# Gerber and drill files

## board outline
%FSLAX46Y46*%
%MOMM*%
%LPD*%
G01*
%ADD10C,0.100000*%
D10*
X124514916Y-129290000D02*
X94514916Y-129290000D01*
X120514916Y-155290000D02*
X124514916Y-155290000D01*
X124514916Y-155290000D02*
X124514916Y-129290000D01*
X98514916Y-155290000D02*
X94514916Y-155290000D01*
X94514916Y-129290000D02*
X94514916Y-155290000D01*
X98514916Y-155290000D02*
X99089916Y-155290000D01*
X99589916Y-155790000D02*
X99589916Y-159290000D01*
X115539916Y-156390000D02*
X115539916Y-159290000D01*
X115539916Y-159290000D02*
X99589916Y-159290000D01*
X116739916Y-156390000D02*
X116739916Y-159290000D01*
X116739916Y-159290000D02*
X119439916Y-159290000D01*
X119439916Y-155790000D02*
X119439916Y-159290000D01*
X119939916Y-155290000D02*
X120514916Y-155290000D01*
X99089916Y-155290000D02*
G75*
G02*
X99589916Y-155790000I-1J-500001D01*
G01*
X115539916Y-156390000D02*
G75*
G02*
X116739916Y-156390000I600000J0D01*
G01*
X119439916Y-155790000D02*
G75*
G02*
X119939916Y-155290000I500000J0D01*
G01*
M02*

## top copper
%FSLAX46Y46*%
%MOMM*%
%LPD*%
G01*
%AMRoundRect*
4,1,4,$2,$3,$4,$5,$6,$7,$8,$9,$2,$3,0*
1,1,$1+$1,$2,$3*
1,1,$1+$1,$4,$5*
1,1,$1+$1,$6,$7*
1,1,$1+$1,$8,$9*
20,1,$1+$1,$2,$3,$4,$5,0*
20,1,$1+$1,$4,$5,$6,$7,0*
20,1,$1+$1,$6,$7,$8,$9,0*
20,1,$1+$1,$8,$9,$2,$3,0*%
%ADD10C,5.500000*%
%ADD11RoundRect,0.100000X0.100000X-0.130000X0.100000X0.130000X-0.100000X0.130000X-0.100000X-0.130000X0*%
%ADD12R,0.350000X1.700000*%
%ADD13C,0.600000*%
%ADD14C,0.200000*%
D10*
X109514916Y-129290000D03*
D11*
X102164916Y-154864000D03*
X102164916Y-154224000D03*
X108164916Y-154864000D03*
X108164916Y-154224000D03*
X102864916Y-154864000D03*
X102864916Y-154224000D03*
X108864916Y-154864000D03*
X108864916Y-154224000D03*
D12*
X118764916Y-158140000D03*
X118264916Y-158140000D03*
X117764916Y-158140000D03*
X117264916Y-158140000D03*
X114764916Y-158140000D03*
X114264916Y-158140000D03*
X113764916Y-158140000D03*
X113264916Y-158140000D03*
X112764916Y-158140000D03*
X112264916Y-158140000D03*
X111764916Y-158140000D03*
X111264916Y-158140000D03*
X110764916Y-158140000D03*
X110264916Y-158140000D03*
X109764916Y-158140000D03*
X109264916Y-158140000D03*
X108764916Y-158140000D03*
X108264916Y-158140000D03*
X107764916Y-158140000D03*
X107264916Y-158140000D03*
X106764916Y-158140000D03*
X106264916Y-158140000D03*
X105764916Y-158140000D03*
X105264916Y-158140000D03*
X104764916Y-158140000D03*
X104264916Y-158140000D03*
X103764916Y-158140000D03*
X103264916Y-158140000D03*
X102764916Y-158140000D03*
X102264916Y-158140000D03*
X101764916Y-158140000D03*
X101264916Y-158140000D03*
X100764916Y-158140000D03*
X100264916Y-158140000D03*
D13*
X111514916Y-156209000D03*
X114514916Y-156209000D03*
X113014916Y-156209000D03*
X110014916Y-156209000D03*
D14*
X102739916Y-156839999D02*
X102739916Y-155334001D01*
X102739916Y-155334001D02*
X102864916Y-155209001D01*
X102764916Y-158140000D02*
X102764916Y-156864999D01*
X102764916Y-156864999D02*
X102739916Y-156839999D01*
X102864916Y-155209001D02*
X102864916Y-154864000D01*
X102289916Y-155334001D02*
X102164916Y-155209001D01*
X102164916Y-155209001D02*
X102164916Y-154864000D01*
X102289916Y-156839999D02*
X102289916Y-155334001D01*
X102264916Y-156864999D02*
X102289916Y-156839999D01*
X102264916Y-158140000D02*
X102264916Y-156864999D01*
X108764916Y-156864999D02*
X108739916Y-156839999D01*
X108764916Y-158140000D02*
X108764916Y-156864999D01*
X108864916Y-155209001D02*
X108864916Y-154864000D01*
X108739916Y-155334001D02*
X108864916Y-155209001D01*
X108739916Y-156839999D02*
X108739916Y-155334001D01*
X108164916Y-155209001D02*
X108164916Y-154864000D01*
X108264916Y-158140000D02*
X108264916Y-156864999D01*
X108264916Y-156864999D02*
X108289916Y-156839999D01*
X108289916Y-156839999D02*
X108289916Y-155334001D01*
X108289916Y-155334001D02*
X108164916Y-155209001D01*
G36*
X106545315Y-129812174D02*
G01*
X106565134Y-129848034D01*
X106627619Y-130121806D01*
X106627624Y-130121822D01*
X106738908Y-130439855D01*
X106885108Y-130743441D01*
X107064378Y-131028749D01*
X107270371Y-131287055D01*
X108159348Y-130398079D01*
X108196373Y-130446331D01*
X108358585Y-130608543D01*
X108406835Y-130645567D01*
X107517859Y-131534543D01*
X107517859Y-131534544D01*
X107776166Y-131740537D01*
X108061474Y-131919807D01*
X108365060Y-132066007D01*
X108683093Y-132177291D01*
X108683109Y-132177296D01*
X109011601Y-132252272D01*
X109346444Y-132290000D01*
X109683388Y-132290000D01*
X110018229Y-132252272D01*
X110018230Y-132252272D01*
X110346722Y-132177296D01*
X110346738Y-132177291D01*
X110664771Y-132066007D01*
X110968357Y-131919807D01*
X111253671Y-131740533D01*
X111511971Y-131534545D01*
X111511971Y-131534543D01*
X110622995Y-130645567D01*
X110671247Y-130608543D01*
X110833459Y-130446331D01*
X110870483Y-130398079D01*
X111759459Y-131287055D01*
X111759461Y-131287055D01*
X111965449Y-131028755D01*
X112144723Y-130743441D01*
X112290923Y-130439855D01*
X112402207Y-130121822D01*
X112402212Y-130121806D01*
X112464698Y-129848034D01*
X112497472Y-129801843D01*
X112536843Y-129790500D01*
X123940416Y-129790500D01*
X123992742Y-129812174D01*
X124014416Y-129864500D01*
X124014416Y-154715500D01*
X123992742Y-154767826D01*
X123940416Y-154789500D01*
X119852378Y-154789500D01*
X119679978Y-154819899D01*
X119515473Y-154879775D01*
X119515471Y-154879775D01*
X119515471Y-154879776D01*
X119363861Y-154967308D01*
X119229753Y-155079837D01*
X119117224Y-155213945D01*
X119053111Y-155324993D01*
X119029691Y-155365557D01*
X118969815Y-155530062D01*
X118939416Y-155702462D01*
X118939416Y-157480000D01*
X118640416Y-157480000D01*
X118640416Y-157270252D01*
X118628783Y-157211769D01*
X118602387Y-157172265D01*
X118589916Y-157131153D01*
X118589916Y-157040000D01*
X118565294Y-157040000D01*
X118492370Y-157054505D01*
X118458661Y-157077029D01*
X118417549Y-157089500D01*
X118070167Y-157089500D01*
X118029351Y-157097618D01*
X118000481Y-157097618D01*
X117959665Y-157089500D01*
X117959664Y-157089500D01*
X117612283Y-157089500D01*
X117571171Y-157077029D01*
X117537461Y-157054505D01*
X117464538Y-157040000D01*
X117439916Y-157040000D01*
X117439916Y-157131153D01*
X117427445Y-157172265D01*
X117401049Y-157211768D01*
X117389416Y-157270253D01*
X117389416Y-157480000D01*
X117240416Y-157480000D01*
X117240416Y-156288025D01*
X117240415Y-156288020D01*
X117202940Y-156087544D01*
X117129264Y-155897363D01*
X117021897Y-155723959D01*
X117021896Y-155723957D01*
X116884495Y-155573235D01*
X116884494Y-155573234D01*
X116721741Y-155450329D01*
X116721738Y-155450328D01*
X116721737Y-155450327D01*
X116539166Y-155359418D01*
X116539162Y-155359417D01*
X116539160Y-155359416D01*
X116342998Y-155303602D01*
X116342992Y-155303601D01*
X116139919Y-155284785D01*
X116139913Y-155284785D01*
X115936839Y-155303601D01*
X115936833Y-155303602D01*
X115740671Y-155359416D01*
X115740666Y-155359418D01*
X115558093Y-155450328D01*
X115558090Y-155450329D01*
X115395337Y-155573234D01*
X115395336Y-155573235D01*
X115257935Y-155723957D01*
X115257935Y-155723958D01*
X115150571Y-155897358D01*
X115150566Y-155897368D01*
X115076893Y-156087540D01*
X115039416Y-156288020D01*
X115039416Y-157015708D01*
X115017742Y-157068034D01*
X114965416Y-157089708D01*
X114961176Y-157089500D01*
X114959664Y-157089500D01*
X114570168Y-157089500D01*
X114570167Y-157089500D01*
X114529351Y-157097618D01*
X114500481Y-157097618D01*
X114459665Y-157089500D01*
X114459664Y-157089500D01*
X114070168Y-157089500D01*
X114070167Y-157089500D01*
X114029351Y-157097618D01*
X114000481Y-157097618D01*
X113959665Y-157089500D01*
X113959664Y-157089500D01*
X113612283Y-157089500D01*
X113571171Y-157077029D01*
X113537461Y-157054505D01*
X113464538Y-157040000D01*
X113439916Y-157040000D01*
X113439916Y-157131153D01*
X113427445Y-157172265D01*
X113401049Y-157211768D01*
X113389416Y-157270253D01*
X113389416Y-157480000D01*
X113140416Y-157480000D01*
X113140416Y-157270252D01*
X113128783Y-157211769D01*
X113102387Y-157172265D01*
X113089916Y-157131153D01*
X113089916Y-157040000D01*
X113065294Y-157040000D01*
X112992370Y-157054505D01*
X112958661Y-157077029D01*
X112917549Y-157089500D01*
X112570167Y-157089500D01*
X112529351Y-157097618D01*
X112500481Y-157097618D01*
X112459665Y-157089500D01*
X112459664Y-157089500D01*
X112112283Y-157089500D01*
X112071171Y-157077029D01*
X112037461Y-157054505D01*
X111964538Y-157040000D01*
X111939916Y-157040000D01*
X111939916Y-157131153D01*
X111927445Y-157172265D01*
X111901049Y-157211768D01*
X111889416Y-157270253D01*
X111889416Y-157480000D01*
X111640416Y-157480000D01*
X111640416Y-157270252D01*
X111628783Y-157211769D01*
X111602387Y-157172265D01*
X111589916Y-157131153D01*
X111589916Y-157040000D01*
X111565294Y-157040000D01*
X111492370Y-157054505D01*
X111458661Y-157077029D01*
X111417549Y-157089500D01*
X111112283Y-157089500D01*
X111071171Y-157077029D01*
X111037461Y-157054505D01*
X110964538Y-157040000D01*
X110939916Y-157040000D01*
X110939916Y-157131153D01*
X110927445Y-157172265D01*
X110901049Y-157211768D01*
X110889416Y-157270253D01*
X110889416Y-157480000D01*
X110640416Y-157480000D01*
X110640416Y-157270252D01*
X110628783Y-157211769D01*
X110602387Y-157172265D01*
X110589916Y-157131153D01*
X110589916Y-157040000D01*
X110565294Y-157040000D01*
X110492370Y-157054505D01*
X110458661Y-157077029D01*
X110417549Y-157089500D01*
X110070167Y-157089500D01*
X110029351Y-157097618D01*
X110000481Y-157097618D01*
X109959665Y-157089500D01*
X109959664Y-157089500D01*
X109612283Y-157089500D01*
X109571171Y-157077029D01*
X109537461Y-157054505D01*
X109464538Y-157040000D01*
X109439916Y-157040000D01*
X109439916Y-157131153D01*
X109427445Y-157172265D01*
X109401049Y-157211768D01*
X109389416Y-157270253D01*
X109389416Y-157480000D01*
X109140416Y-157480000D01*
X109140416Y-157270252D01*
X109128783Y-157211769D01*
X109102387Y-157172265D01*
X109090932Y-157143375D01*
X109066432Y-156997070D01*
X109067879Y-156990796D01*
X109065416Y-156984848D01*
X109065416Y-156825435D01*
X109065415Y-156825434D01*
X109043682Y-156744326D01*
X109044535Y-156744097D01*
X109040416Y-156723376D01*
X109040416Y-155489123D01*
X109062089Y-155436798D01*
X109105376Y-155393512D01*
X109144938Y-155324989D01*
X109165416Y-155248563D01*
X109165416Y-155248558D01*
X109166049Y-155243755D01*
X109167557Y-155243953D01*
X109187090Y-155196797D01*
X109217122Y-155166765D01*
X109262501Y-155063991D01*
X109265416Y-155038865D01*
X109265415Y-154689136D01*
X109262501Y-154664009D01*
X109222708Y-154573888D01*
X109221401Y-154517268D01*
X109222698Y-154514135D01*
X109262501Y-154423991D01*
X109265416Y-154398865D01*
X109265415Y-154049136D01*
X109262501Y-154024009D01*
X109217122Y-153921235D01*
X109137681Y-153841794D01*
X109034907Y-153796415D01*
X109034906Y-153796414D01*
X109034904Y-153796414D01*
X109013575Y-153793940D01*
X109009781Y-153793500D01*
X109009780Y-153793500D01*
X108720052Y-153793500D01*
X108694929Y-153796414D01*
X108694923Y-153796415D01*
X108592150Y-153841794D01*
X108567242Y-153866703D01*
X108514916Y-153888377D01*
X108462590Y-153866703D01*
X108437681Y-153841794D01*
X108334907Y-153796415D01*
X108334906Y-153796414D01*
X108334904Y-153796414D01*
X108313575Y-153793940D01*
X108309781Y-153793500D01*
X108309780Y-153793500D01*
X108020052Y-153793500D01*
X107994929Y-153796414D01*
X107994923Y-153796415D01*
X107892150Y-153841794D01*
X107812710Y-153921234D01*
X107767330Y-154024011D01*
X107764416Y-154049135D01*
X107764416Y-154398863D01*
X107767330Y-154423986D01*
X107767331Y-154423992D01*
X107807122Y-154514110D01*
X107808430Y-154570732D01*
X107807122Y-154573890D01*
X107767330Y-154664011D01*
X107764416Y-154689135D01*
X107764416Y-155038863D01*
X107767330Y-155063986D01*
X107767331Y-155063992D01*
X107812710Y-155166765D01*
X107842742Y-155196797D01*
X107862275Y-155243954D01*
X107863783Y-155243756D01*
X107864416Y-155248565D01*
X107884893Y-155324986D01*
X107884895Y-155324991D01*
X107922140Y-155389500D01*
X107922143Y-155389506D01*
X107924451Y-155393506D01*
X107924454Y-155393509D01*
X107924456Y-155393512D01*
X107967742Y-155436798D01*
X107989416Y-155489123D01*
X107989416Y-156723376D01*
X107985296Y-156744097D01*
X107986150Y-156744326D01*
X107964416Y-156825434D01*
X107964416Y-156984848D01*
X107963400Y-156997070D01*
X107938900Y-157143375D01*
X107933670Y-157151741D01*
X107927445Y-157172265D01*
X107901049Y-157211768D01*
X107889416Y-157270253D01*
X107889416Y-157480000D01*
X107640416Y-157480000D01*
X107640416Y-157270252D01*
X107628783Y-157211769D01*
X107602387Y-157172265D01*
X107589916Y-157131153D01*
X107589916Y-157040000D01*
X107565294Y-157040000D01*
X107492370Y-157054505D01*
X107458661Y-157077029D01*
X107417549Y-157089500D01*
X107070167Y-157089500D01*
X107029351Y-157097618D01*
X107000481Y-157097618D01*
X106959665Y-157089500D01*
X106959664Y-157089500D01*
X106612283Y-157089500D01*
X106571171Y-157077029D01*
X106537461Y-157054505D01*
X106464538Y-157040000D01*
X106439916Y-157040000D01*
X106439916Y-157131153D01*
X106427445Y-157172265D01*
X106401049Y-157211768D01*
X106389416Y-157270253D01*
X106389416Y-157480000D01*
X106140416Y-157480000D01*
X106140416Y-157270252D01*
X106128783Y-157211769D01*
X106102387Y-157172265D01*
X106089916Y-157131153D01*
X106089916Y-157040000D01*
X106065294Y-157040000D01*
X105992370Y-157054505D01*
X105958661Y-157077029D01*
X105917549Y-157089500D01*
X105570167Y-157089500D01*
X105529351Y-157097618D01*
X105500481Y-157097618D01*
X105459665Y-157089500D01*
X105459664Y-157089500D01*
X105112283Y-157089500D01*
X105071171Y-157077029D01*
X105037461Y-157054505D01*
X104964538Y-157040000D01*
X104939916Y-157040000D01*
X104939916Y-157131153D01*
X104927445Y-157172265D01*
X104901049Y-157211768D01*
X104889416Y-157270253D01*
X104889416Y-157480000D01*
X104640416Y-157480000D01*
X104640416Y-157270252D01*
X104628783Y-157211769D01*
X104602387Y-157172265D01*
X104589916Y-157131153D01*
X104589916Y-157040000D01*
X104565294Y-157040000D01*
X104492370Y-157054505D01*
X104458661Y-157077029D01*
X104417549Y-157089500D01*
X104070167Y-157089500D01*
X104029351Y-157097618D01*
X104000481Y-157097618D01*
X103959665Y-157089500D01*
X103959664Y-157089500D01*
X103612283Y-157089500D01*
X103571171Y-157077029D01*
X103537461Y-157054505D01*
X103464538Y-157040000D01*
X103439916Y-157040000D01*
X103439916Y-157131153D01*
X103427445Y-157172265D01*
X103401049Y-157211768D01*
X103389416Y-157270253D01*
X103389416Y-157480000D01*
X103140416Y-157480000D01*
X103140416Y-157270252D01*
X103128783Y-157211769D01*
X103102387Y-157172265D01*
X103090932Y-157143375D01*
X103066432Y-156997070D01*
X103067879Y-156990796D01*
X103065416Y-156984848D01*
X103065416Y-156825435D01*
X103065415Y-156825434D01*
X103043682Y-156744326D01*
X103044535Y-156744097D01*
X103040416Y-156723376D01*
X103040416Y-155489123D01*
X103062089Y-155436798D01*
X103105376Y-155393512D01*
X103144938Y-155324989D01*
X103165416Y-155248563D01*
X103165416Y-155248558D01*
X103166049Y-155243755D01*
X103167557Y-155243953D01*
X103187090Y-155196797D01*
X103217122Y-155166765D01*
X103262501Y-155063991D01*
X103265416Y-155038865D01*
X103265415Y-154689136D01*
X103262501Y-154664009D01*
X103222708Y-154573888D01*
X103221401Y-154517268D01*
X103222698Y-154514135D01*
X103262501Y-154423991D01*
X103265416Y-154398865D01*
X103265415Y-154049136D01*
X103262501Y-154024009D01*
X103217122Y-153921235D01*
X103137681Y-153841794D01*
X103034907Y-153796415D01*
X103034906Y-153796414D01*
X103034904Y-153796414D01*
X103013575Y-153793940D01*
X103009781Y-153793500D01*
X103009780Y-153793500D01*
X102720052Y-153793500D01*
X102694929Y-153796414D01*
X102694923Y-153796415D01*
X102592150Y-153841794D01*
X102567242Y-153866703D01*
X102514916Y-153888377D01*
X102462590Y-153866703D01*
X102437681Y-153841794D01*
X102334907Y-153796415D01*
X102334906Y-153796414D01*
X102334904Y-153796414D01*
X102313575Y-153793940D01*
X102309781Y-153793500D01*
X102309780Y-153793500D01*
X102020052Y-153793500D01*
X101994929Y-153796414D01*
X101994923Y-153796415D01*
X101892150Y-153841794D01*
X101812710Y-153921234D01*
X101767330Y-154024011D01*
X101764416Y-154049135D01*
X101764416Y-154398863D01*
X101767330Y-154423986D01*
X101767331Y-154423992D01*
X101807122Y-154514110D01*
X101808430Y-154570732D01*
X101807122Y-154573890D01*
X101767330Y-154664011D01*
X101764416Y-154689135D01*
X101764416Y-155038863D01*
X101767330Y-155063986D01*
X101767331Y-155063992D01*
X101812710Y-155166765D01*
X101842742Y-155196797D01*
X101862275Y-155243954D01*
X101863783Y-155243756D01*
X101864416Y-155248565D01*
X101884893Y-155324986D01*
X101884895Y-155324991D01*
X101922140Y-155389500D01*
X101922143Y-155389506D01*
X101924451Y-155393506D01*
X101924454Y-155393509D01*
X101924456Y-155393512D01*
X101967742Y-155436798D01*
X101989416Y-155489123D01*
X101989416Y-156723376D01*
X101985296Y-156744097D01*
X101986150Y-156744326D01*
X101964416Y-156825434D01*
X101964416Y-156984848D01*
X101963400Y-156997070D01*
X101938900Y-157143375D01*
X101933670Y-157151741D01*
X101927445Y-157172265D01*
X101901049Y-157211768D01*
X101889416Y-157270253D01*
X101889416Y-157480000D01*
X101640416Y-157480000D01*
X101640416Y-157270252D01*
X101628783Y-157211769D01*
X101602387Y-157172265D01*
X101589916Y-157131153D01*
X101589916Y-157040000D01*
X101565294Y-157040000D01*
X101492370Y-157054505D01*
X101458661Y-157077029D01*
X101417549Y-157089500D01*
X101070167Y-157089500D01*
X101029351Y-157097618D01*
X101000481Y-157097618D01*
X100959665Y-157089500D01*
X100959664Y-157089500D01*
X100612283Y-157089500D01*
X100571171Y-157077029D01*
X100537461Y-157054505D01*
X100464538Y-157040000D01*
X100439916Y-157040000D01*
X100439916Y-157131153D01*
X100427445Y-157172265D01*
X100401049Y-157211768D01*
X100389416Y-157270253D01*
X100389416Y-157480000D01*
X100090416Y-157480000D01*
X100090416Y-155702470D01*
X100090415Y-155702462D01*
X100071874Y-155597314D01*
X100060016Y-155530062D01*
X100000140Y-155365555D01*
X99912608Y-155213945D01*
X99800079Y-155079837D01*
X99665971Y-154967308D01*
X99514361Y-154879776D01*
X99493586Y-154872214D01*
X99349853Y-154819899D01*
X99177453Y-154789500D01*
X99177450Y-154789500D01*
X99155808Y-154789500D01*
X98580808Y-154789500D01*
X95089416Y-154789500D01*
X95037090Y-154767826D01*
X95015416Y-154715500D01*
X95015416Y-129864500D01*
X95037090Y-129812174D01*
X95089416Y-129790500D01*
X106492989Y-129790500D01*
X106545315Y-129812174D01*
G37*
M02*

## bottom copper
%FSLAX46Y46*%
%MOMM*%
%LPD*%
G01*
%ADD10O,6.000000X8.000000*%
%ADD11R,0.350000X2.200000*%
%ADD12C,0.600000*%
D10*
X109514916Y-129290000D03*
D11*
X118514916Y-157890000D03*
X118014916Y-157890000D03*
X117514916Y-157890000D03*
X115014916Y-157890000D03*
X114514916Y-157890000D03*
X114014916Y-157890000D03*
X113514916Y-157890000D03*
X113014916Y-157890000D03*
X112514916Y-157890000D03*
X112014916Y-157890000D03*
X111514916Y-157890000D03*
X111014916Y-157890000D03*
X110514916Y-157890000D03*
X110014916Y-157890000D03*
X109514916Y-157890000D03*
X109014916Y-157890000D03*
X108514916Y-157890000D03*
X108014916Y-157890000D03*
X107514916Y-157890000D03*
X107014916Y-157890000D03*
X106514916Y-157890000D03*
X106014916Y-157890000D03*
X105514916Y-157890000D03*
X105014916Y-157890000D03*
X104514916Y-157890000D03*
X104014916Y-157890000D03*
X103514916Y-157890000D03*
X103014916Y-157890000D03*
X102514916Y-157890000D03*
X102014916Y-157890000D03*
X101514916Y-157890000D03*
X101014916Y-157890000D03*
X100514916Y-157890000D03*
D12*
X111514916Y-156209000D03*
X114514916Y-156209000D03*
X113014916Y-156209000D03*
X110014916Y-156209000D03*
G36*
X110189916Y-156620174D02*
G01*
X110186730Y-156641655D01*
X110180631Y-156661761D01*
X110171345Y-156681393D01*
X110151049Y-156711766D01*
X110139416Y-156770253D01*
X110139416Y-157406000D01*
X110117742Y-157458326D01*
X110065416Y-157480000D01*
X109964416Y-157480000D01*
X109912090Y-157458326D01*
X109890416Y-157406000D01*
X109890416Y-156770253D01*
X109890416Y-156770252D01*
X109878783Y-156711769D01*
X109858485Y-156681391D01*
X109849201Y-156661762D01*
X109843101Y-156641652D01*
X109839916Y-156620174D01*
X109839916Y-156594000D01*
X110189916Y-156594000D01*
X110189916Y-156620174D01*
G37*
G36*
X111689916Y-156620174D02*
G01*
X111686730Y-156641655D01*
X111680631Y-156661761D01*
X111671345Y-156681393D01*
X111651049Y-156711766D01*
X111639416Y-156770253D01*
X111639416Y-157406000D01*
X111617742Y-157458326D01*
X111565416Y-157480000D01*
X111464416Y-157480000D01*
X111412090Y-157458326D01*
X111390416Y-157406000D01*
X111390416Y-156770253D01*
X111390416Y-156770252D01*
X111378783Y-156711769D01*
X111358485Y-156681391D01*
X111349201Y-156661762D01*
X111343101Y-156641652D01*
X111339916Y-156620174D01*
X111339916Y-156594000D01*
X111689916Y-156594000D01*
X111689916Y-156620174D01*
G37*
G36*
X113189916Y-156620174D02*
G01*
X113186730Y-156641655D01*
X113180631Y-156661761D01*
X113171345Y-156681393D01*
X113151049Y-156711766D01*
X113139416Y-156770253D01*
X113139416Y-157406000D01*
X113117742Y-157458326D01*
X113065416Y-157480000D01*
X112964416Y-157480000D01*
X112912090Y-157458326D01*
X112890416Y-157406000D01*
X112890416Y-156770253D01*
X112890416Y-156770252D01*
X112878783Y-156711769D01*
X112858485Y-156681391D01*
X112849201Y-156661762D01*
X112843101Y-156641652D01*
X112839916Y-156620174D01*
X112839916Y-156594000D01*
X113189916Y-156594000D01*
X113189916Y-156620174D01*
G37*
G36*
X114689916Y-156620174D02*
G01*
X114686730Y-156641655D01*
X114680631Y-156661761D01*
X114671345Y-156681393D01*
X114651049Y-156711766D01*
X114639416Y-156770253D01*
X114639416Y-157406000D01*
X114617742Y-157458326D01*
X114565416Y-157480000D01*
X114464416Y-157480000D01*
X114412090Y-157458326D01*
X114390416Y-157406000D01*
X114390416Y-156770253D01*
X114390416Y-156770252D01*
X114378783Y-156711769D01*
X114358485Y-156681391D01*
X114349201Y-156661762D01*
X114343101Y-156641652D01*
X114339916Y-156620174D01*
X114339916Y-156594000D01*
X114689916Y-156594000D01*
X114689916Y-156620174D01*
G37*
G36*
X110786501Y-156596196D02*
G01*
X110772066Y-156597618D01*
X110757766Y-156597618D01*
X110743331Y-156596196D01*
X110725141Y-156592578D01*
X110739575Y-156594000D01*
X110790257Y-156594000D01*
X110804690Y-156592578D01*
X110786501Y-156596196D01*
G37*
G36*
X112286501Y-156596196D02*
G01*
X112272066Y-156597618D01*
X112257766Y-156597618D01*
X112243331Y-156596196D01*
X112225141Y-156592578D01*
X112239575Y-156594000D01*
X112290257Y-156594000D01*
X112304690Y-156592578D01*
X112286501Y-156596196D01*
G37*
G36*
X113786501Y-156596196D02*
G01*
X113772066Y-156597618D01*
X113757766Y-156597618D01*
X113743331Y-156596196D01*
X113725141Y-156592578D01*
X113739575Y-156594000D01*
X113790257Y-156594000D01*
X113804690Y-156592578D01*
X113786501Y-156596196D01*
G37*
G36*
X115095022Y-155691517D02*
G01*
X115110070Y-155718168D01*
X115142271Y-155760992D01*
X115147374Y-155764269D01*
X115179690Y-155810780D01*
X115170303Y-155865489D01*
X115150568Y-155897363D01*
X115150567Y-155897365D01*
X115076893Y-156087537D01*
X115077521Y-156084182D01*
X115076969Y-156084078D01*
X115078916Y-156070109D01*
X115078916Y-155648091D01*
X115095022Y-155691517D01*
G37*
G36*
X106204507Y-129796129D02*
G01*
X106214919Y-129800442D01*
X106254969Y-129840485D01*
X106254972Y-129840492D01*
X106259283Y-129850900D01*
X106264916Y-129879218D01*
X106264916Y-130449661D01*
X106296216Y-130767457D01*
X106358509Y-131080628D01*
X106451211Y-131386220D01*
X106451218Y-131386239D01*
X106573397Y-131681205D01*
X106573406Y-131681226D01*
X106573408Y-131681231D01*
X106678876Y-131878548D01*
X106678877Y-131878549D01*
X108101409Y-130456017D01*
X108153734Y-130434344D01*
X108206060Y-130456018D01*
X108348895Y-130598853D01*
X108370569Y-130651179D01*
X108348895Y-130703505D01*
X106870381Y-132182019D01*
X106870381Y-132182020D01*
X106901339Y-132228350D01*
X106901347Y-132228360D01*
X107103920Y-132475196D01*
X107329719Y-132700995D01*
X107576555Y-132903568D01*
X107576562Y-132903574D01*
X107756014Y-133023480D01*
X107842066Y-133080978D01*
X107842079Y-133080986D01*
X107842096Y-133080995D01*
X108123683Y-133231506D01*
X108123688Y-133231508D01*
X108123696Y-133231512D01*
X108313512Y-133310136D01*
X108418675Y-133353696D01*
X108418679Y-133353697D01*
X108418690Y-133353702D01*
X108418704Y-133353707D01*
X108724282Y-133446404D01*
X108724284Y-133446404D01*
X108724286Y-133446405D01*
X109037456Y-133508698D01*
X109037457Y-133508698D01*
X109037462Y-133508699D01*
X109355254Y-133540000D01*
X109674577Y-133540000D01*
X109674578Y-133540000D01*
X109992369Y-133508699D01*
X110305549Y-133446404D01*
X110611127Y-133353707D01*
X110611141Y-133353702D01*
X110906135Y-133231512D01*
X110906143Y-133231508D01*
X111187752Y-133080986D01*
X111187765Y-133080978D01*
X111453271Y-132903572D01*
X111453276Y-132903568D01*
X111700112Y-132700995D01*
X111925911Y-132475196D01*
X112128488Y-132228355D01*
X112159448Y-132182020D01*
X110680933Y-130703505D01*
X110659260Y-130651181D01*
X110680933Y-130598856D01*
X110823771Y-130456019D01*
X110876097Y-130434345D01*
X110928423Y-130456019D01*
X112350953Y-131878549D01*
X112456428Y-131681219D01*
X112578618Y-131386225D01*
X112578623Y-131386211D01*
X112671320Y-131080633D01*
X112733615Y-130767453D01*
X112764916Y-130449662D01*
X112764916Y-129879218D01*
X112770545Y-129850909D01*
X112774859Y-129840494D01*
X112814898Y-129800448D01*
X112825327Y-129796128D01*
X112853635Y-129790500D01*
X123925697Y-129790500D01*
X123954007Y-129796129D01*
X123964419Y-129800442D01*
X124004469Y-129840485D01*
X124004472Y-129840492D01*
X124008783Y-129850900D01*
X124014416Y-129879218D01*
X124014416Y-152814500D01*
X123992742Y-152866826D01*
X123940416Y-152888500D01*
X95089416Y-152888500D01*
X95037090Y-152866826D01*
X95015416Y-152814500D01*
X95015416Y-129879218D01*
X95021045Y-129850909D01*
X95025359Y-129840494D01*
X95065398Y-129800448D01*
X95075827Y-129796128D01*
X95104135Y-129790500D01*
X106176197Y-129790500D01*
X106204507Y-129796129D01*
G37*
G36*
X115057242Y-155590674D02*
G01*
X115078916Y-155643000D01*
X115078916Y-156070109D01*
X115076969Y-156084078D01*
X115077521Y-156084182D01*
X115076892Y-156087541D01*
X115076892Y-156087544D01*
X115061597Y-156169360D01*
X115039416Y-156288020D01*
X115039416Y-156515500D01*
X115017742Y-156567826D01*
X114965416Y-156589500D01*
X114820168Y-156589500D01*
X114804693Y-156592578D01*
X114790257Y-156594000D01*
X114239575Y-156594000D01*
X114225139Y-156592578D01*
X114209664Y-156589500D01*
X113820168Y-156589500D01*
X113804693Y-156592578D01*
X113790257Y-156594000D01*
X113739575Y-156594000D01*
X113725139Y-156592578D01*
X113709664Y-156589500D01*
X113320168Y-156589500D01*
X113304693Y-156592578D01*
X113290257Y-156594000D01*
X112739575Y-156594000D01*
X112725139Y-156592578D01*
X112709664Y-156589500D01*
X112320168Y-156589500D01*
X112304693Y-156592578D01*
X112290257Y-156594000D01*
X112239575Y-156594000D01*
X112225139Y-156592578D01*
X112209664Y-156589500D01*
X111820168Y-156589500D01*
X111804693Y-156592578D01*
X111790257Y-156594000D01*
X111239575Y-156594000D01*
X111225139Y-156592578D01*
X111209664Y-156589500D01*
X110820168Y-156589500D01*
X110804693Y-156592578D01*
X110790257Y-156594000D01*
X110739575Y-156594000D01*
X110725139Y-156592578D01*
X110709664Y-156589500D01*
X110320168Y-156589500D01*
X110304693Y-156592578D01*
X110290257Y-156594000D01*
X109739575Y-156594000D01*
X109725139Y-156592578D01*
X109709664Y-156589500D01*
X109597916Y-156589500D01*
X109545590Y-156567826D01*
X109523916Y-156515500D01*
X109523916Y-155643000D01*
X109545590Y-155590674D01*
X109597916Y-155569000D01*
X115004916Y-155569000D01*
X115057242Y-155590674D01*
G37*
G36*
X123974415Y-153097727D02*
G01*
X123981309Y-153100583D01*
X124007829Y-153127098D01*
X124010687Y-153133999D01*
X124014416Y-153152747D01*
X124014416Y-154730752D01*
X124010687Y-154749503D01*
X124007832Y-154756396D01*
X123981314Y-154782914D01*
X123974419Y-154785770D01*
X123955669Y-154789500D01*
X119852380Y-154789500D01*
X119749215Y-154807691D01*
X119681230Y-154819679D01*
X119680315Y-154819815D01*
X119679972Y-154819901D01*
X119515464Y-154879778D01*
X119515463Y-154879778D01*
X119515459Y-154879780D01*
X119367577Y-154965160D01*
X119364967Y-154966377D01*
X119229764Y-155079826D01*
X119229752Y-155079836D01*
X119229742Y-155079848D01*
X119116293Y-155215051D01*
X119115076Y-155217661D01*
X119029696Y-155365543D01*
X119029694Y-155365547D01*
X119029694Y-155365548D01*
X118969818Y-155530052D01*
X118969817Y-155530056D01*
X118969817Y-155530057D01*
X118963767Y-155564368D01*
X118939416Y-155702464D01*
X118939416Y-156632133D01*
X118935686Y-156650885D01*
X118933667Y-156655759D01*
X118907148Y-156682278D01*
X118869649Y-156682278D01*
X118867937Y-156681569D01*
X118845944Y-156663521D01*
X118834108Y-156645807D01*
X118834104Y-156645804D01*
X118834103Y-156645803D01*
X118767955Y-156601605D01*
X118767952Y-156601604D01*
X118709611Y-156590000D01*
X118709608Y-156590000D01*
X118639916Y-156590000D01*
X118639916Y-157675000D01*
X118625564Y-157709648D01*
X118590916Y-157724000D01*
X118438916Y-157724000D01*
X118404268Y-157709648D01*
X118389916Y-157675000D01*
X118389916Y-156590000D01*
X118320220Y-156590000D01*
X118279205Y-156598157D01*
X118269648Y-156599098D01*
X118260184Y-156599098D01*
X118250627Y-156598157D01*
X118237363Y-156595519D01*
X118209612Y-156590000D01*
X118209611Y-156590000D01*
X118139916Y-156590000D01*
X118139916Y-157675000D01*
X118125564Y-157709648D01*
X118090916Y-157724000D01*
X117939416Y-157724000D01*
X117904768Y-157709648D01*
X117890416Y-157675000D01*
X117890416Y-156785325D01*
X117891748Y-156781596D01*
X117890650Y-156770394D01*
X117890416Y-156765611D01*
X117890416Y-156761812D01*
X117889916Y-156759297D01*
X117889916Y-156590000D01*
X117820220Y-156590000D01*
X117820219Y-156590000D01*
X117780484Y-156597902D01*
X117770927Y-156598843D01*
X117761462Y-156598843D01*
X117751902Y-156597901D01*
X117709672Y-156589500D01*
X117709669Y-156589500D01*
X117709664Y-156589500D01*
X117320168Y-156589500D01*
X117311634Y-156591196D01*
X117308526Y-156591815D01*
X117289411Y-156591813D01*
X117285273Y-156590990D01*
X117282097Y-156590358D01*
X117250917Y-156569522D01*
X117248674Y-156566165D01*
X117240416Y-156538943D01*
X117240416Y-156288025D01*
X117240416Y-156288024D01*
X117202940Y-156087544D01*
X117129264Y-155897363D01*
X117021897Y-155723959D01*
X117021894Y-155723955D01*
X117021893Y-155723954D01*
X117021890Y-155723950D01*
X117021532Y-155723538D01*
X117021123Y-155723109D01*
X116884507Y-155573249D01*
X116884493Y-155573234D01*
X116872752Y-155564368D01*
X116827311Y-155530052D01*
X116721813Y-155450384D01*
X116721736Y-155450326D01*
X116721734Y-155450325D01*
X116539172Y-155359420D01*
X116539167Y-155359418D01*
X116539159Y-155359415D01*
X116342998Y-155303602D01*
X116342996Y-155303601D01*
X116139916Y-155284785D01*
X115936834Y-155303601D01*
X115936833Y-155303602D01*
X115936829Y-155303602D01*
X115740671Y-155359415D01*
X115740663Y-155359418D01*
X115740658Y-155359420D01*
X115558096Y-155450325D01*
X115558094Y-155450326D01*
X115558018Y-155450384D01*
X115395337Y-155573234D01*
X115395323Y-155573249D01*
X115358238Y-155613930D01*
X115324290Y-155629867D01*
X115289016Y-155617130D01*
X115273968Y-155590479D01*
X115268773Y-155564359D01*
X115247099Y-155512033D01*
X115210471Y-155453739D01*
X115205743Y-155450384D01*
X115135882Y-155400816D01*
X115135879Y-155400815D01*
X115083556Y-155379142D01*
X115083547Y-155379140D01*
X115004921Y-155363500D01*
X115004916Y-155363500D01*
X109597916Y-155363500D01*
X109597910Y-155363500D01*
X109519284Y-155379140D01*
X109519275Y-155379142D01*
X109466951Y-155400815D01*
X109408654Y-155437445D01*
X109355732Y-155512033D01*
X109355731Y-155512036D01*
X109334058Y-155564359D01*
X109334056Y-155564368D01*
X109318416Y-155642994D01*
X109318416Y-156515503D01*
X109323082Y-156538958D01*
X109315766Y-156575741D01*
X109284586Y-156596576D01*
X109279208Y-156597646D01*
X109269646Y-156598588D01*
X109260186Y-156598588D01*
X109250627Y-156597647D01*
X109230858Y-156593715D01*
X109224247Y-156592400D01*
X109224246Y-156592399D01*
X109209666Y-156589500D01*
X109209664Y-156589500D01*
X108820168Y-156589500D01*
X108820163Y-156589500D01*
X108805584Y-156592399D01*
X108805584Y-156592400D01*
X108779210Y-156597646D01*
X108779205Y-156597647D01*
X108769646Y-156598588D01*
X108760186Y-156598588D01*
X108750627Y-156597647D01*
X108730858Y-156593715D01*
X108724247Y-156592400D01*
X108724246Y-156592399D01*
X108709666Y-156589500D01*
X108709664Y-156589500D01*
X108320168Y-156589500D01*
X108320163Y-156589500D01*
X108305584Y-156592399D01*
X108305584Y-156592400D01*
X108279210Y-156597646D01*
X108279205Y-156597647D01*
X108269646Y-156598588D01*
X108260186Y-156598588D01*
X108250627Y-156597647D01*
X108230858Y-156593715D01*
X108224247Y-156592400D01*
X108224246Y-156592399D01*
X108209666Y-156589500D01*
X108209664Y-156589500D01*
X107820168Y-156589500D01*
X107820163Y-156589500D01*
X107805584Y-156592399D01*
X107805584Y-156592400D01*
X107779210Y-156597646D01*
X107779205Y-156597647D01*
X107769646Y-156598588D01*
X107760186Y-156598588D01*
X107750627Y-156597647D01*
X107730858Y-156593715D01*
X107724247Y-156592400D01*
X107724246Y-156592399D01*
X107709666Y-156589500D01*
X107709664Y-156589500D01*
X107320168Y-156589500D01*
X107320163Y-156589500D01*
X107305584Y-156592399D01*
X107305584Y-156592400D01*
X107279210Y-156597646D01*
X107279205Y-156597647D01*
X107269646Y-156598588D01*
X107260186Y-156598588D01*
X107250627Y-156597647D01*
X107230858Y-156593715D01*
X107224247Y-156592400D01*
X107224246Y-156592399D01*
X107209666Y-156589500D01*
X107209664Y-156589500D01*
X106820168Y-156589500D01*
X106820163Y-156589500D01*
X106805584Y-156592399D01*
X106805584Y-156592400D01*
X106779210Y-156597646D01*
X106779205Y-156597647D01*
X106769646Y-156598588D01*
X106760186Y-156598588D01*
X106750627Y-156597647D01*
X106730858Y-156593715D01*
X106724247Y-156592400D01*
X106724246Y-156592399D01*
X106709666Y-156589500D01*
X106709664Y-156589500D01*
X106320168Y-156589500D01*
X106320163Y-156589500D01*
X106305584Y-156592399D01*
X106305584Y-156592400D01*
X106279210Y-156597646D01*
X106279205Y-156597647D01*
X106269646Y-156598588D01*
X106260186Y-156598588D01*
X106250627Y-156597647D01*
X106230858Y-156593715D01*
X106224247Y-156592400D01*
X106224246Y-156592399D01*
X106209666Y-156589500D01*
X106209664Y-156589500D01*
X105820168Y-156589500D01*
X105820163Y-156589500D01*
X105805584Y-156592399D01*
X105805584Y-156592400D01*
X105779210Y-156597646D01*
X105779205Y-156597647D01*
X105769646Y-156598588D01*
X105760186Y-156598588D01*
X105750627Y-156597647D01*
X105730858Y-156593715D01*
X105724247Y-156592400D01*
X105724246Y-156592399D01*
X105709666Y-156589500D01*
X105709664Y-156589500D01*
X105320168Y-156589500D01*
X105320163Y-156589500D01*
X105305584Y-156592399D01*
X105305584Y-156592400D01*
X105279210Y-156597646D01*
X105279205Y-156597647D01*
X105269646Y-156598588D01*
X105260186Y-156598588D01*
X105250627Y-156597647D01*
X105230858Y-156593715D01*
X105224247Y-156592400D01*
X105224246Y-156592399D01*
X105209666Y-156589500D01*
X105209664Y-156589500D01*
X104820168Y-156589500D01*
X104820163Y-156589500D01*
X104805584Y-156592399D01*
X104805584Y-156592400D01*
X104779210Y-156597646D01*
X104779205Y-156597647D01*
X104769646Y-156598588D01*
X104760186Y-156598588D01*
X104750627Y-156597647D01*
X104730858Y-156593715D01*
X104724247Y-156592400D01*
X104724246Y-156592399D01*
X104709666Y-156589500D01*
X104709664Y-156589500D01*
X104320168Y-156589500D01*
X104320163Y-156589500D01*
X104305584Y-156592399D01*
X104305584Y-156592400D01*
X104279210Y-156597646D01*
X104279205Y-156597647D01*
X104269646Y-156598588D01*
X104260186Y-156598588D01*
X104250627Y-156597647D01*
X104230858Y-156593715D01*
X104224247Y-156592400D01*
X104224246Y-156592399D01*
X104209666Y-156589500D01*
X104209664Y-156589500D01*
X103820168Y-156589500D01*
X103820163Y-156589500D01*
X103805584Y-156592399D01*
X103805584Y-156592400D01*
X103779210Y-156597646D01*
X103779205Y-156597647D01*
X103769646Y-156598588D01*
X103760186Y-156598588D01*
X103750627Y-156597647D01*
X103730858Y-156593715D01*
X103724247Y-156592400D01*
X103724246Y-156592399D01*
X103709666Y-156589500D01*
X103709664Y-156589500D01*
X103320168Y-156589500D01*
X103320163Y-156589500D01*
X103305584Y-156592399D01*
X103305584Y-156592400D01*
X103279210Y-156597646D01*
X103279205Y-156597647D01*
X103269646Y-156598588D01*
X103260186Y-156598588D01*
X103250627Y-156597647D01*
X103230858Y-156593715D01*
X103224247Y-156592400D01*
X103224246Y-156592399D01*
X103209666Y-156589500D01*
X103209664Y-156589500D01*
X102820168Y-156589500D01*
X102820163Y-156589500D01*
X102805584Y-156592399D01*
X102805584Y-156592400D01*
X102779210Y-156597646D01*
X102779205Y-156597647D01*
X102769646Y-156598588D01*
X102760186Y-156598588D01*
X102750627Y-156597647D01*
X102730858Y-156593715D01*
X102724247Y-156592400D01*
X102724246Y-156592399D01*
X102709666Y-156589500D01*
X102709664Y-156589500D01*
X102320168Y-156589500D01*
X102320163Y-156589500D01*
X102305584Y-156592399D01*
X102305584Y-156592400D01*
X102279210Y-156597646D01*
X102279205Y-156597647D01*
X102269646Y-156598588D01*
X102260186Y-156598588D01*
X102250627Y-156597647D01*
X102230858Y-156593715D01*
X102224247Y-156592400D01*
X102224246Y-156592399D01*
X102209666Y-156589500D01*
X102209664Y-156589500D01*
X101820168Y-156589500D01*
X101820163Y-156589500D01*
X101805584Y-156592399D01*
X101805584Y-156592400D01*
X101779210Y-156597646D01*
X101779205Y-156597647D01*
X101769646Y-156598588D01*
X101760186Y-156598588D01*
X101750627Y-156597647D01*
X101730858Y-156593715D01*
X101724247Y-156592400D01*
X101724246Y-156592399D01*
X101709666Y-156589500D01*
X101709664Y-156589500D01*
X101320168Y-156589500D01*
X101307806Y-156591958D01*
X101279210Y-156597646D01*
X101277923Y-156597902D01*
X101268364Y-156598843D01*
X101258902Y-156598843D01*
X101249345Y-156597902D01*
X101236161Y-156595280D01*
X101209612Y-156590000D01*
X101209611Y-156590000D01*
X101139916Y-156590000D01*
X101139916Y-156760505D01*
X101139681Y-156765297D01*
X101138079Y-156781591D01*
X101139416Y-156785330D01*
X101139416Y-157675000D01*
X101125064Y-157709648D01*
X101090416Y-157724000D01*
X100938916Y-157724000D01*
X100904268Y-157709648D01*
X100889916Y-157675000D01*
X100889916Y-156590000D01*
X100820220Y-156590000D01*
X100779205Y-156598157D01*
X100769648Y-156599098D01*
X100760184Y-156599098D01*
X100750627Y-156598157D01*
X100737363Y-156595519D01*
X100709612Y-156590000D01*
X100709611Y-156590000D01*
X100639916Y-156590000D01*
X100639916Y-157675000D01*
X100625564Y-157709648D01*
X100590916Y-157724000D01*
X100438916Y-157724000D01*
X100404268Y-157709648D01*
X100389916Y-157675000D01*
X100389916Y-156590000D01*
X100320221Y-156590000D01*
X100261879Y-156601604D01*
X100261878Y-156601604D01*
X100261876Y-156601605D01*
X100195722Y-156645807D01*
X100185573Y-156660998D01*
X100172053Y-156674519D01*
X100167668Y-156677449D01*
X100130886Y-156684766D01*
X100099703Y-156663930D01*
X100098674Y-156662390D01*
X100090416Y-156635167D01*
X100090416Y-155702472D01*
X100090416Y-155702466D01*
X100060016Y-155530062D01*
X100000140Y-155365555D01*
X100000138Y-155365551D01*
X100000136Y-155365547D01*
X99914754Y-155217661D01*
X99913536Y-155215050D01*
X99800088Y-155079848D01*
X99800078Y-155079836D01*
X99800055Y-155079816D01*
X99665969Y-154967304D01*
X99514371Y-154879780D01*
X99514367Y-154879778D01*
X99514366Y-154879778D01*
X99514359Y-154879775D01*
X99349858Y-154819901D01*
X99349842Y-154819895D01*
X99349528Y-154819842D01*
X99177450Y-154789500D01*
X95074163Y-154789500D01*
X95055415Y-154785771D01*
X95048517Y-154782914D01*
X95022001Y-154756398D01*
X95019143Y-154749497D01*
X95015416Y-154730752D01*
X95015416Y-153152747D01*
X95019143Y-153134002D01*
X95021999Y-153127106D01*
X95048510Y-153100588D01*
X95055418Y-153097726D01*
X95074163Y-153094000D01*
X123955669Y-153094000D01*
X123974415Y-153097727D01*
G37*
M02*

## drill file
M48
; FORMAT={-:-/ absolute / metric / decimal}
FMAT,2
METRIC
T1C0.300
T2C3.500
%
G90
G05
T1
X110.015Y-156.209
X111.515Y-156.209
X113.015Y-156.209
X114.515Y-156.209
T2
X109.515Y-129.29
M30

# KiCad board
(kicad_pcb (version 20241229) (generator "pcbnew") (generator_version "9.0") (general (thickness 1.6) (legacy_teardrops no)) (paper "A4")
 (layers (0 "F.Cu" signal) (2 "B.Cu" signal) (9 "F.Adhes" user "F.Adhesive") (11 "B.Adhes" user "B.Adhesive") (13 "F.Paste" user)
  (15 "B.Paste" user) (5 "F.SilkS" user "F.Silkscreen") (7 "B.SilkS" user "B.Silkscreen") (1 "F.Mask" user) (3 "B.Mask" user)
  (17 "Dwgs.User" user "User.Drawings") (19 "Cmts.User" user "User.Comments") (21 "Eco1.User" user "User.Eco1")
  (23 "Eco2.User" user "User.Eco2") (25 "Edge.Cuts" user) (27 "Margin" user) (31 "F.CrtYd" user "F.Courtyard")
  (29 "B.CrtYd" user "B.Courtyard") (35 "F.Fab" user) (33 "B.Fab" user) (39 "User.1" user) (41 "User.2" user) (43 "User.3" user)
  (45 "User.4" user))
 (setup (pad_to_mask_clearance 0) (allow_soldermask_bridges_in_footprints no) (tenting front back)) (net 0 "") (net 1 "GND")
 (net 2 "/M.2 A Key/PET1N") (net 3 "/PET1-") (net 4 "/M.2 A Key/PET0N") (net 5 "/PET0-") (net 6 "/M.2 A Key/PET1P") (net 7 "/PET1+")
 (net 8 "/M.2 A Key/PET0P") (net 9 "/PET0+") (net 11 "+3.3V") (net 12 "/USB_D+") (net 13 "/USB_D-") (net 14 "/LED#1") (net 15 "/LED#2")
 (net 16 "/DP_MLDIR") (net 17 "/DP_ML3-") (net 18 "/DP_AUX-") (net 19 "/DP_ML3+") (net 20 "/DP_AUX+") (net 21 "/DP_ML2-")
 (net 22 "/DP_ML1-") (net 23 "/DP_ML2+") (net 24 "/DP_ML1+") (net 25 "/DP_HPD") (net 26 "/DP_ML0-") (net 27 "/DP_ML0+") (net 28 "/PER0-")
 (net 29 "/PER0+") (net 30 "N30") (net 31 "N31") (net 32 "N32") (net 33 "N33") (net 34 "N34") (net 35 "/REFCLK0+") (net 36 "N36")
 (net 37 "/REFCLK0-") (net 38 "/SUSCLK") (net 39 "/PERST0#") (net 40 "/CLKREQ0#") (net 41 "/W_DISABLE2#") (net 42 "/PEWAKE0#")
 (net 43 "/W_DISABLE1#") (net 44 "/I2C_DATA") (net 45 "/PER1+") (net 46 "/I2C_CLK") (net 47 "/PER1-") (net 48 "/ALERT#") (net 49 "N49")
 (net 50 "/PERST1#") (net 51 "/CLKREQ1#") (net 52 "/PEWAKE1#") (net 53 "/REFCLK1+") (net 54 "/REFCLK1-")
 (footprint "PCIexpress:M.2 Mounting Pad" (layer "F.Cu") (at 109.514916 129.29)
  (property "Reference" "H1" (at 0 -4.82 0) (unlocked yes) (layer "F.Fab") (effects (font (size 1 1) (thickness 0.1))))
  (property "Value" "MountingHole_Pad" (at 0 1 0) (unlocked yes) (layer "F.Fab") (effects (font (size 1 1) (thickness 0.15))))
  (pad "1" thru_hole circle (at 0 0) (size 5.5 5.5) (drill 3.5) (layers "*.Cu" "*.Mask") (remove_unused_layers no) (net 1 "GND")
   (padstack (mode front_inner_back)
    (layer "Inner" (shape circle) (size 5.5 5.5) (zone_connect -1))
    (layer "B.Cu" (shape oval) (size 6 8) (thermal_bridge_angle 45) (zone_connect -1)))))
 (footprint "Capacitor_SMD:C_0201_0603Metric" (layer "F.Cu") (at 102.164916 154.544 90)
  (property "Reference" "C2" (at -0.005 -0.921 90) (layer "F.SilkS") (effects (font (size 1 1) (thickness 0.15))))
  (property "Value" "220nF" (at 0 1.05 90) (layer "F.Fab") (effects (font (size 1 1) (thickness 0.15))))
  (pad "" smd roundrect (at -0.345 0 90) (size 0.318 0.36) (layers "F.Paste") (roundrect_rratio 0.25))
  (pad "" smd roundrect (at 0.345 0 90) (size 0.318 0.36) (layers "F.Paste") (roundrect_rratio 0.25))
  (pad "1" smd roundrect (at -0.32 0 90) (size 0.46 0.4) (layers "F.Cu" "F.Mask") (roundrect_rratio 0.25) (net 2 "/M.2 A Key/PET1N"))
  (pad "2" smd roundrect (at 0.32 0 90) (size 0.46 0.4) (layers "F.Cu" "F.Mask") (roundrect_rratio 0.25) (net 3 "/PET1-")))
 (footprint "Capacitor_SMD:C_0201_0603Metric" (layer "F.Cu") (at 108.164916 154.544 90)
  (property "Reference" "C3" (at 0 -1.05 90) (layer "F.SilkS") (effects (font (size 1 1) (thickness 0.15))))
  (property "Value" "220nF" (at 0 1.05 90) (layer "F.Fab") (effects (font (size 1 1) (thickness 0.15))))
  (pad "" smd roundrect (at -0.345 0 90) (size 0.318 0.36) (layers "F.Paste") (roundrect_rratio 0.25))
  (pad "" smd roundrect (at 0.345 0 90) (size 0.318 0.36) (layers "F.Paste") (roundrect_rratio 0.25))
  (pad "1" smd roundrect (at -0.32 0 90) (size 0.46 0.4) (layers "F.Cu" "F.Mask") (roundrect_rratio 0.25) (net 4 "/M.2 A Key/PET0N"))
  (pad "2" smd roundrect (at 0.32 0 90) (size 0.46 0.4) (layers "F.Cu" "F.Mask") (roundrect_rratio 0.25) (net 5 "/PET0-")))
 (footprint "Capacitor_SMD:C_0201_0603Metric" (layer "F.Cu") (at 102.864916 154.544 90)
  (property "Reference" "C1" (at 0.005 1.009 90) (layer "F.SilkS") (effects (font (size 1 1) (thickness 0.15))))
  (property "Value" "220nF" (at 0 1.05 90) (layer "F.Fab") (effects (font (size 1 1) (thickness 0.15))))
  (pad "" smd roundrect (at -0.345 0 90) (size 0.318 0.36) (layers "F.Paste") (roundrect_rratio 0.25))
  (pad "" smd roundrect (at 0.345 0 90) (size 0.318 0.36) (layers "F.Paste") (roundrect_rratio 0.25))
  (pad "1" smd roundrect (at -0.32 0 90) (size 0.46 0.4) (layers "F.Cu" "F.Mask") (roundrect_rratio 0.25) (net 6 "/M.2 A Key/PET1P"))
  (pad "2" smd roundrect (at 0.32 0 90) (size 0.46 0.4) (layers "F.Cu" "F.Mask") (roundrect_rratio 0.25) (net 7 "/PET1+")))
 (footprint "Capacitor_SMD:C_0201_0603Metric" (layer "F.Cu") (at 108.864916 154.544 90)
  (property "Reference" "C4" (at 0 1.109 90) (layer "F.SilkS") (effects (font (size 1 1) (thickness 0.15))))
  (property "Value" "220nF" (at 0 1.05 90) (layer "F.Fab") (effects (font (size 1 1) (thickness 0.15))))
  (pad "" smd roundrect (at -0.345 0 90) (size 0.318 0.36) (layers "F.Paste") (roundrect_rratio 0.25))
  (pad "" smd roundrect (at 0.345 0 90) (size 0.318 0.36) (layers "F.Paste") (roundrect_rratio 0.25))
  (pad "1" smd roundrect (at -0.32 0 90) (size 0.46 0.4) (layers "F.Cu" "F.Mask") (roundrect_rratio 0.25) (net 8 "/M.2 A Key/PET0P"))
  (pad "2" smd roundrect (at 0.32 0 90) (size 0.46 0.4) (layers "F.Cu" "F.Mask") (roundrect_rratio 0.25) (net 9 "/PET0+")))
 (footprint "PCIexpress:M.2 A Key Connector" (layer "F.Cu") (at 109.514916 158.18)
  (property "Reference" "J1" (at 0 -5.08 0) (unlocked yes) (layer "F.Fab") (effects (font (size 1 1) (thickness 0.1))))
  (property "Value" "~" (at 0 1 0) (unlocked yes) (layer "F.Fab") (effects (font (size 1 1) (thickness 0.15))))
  (fp_line (start -11 -2.89) (end -10.425 -2.89) (stroke (width 0.1) (type default)) (layer "Edge.Cuts") (net 10))
  (fp_line (start -9.925 -2.39) (end -9.925 1.11) (stroke (width 0.1) (type default)) (layer "Edge.Cuts") (net 10))
  (fp_line (start 6.025 -1.79) (end 6.025 1.11) (stroke (width 0.1) (type default)) (layer "Edge.Cuts") (net 10))
  (fp_line (start 6.025 1.11) (end -9.925 1.11) (stroke (width 0.1) (type default)) (layer "Edge.Cuts") (net 10))
  (fp_line (start 7.225 -1.79) (end 7.225 1.11) (stroke (width 0.1) (type default)) (layer "Edge.Cuts") (net 10))
  (fp_line (start 7.225 1.11) (end 9.925 1.11) (stroke (width 0.1) (type default)) (layer "Edge.Cuts") (net 10))
  (fp_line (start 9.925 -2.39) (end 9.925 1.11) (stroke (width 0.1) (type default)) (layer "Edge.Cuts") (net 10))
  (fp_line (start 10.425 -2.89) (end 11 -2.89) (stroke (width 0.1) (type default)) (layer "Edge.Cuts") (net 10))
  (fp_arc (start -10.425 -2.89) (mid -10.071447 -2.743553) (end -9.925 -2.39) (stroke (width 0.1) (type default)) (layer "Edge.Cuts")
   (net 10))
  (fp_arc (start 6.025 -1.79) (mid 6.625 -2.39) (end 7.225 -1.79) (stroke (width 0.1) (type default)) (layer "Edge.Cuts") (net 10))
  (fp_arc (start 9.925 -2.39) (mid 10.071447 -2.743553) (end 10.425 -2.89) (stroke (width 0.1) (type default)) (layer "Edge.Cuts") (net 10))
  (pad "1" smd rect (at 9.25 -0.04 180) (size 0.35 1.7) (layers "F.Cu") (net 1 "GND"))
  (pad "2" smd rect (at 9 -0.29 180) (size 0.35 2.2) (layers "B.Cu") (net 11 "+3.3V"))
  (pad "3" smd rect (at 8.75 -0.04 180) (size 0.35 1.7) (layers "F.Cu") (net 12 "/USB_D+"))
  (pad "4" smd rect (at 8.5 -0.29 180) (size 0.35 2.2) (layers "B.Cu") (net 11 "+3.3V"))
  (pad "5" smd rect (at 8.25 -0.04 180) (size 0.35 1.7) (layers "F.Cu") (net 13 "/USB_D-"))
  (pad "6" smd rect (at 8 -0.29 180) (size 0.35 2.2) (layers "B.Cu") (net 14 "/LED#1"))
  (pad "7" smd rect (at 7.75 -0.04 180) (size 0.35 1.7) (layers "F.Cu") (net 1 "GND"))
  (pad "16" smd rect (at 5.5 -0.29 180) (size 0.35 2.2) (layers "B.Cu") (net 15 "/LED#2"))
  (pad "17" smd rect (at 5.25 -0.04 180) (size 0.35 1.7) (layers "F.Cu") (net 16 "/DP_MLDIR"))
  (pad "18" smd rect (at 5 -0.29 180) (size 0.35 2.2) (layers "B.Cu") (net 1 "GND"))
  (pad "19" smd rect (at 4.75 -0.04 180) (size 0.35 1.7) (layers "F.Cu") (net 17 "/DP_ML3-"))
  (pad "20" smd rect (at 4.5 -0.29 180) (size 0.35 2.2) (layers "B.Cu") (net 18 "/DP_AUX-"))
  (pad "21" smd rect (at 4.25 -0.04 180) (size 0.35 1.7) (layers "F.Cu") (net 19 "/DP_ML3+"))
  (pad "22" smd rect (at 4 -0.29 180) (size 0.35 2.2) (layers "B.Cu") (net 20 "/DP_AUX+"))
  (pad "23" smd rect (at 3.75 -0.04 180) (size 0.35 1.7) (layers "F.Cu") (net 1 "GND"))
  (pad "24" smd rect (at 3.5 -0.29 180) (size 0.35 2.2) (layers "B.Cu") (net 1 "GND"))
  (pad "25" smd rect (at 3.25 -0.04 180) (size 0.35 1.7) (layers "F.Cu") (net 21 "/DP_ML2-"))
  (pad "26" smd rect (at 3 -0.29 180) (size 0.35 2.2) (layers "B.Cu") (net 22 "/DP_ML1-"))
  (pad "27" smd rect (at 2.75 -0.04 180) (size 0.35 1.7) (layers "F.Cu") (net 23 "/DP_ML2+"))
  (pad "28" smd rect (at 2.5 -0.29 180) (size 0.35 2.2) (layers "B.Cu") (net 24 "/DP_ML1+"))
  (pad "29" smd rect (at 2.25 -0.04 180) (size 0.35 1.7) (layers "F.Cu") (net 1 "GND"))
  (pad "30" smd rect (at 2 -0.29 180) (size 0.35 2.2) (layers "B.Cu") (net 1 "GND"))
  (pad "31" smd rect (at 1.75 -0.04 180) (size 0.35 1.7) (layers "F.Cu") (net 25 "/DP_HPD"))
  (pad "32" smd rect (at 1.5 -0.29 180) (size 0.35 2.2) (layers "B.Cu") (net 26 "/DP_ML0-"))
  (pad "33" smd rect (at 1.25 -0.04 180) (size 0.35 1.7) (layers "F.Cu") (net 1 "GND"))
  (pad "34" smd rect (at 1 -0.29 180) (size 0.35 2.2) (layers "B.Cu") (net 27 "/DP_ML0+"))
  (pad "35" smd rect (at 0.75 -0.04 180) (size 0.35 1.7) (layers "F.Cu") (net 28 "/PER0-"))
  (pad "36" smd rect (at 0.5 -0.29 180) (size 0.35 2.2) (layers "B.Cu") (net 1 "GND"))
  (pad "37" smd rect (at 0.25 -0.04 180) (size 0.35 1.7) (layers "F.Cu") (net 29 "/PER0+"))
  (pad "38" smd rect (at 0 -0.29 180) (size 0.35 2.2) (layers "B.Cu") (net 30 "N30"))
  (pad "39" smd rect (at -0.25 -0.04 180) (size 0.35 1.7) (layers "F.Cu") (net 1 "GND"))
  (pad "40" smd rect (at -0.5 -0.29 180) (size 0.35 2.2) (layers "B.Cu") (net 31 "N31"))
  (pad "41" smd rect (at -0.75 -0.04 180) (size 0.35 1.7) (layers "F.Cu") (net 8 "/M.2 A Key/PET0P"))
  (pad "42" smd rect (at -1 -0.29 180) (size 0.35 2.2) (layers "B.Cu") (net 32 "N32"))
  (pad "43" smd rect (at -1.25 -0.04 180) (size 0.35 1.7) (layers "F.Cu") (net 4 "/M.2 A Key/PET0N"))
  (pad "44" smd rect (at -1.5 -0.29 180) (size 0.35 2.2) (layers "B.Cu") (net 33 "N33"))
  (pad "45" smd rect (at -1.75 -0.04 180) (size 0.35 1.7) (layers "F.Cu") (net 1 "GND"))
  (pad "46" smd rect (at -2 -0.29 180) (size 0.35 2.2) (layers "B.Cu") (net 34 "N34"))
  (pad "47" smd rect (at -2.25 -0.04 180) (size 0.35 1.7) (layers "F.Cu") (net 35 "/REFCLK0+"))
  (pad "48" smd rect (at -2.5 -0.29 180) (size 0.35 2.2) (layers "B.Cu") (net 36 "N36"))
  (pad "49" smd rect (at -2.75 -0.04 180) (size 0.35 1.7) (layers "F.Cu") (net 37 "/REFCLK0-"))
  (pad "50" smd rect (at -3 -0.29 180) (size 0.35 2.2) (layers "B.Cu") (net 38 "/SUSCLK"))
  (pad "51" smd rect (at -3.25 -0.04 180) (size 0.35 1.7) (layers "F.Cu") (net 1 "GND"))
  (pad "52" smd rect (at -3.5 -0.29 180) (size 0.35 2.2) (layers "B.Cu") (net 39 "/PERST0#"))
  (pad "53" smd rect (at -3.75 -0.04 180) (size 0.35 1.7) (layers "F.Cu") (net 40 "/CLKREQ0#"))
  (pad "54" smd rect (at -4 -0.29 180) (size 0.35 2.2) (layers "B.Cu") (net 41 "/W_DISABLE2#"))
  (pad "55" smd rect (at -4.25 -0.04 180) (size 0.35 1.7) (layers "F.Cu") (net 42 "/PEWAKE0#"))
  (pad "56" smd rect (at -4.5 -0.29 180) (size 0.35 2.2) (layers "B.Cu") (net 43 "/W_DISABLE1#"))
  (pad "57" smd rect (at -4.75 -0.04 180) (size 0.35 1.7) (layers "F.Cu") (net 1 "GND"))
  (pad "58" smd rect (at -5 -0.29 180) (size 0.35 2.2) (layers "B.Cu") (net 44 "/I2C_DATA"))
  (pad "59" smd rect (at -5.25 -0.04 180) (size 0.35 1.7) (layers "F.Cu") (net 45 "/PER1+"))
  (pad "60" smd rect (at -5.5 -0.29 180) (size 0.35 2.2) (layers "B.Cu") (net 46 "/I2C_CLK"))
  (pad "61" smd rect (at -5.75 -0.04 180) (size 0.35 1.7) (layers "F.Cu") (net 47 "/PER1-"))
  (pad "62" smd rect (at -6 -0.29 180) (size 0.35 2.2) (layers "B.Cu") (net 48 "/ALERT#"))
  (pad "63" smd rect (at -6.25 -0.04 180) (size 0.35 1.7) (layers "F.Cu") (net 1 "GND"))
  (pad "64" smd rect (at -6.5 -0.29 180) (size 0.35 2.2) (layers "B.Cu") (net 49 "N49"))
  (pad "65" smd rect (at -6.75 -0.04 180) (size 0.35 1.7) (layers "F.Cu") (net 6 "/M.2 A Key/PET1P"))
  (pad "66" smd rect (at -7 -0.29 180) (size 0.35 2.2) (layers "B.Cu") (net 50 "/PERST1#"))
  (pad "67" smd rect (at -7.25 -0.04 180) (size 0.35 1.7) (layers "F.Cu") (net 2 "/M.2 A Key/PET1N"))
  (pad "68" smd rect (at -7.5 -0.29 180) (size 0.35 2.2) (layers "B.Cu") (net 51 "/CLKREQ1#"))
  (pad "69" smd rect (at -7.75 -0.04 180) (size 0.35 1.7) (layers "F.Cu") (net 1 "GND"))
  (pad "70" smd rect (at -8 -0.29 180) (size 0.35 2.2) (layers "B.Cu") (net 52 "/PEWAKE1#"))
  (pad "71" smd rect (at -8.25 -0.04 180) (size 0.35 1.7) (layers "F.Cu") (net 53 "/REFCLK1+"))
  (pad "72" smd rect (at -8.5 -0.29 180) (size 0.35 2.2) (layers "B.Cu") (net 11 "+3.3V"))
  (pad "73" smd rect (at -8.75 -0.04 180) (size 0.35 1.7) (layers "F.Cu") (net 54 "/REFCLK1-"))
  (pad "74" smd rect (at -9 -0.29 180) (size 0.35 2.2) (layers "B.Cu") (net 11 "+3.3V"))
  (pad "75" smd rect (at -9.25 -0.04 180) (size 0.35 1.7) (layers "F.Cu") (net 1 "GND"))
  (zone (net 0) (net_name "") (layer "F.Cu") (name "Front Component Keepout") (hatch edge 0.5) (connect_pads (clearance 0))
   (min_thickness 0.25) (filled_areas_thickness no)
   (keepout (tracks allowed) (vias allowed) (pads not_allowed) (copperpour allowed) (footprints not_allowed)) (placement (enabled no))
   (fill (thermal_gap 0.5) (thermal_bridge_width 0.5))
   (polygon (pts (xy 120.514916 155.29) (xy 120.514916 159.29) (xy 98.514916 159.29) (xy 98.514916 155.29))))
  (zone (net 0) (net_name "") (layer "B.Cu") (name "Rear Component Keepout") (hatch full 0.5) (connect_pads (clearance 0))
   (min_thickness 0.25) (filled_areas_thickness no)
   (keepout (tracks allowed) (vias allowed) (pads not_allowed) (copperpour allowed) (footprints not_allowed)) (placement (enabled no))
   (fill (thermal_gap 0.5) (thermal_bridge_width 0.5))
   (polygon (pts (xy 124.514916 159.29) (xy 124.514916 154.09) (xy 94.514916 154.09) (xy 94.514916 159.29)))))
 (gr_line (start 124.514916 129.29) (end 94.514916 129.29) (stroke (width 0.1) (type solid)) (layer "Edge.Cuts"))
 (gr_line (start 120.514916 155.29) (end 124.514916 155.29) (stroke (width 0.1) (type default)) (layer "Edge.Cuts"))
 (gr_line (start 124.514916 155.29) (end 124.514916 129.29) (stroke (width 0.1) (type default)) (layer "Edge.Cuts"))
 (gr_line (start 98.514916 155.29) (end 94.514916 155.29) (stroke (width 0.1) (type default)) (layer "Edge.Cuts"))
 (gr_line (start 94.514916 129.29) (end 94.514916 155.29) (stroke (width 0.1) (type default)) (layer "Edge.Cuts"))
 (via (at 111.514916 156.209) (size 0.6) (drill 0.3) (layers "F.Cu" "B.Cu") (free yes) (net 1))
 (via (at 114.514916 156.209) (size 0.6) (drill 0.3) (layers "F.Cu" "B.Cu") (free yes) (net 1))
 (via (at 113.014916 156.209) (size 0.6) (drill 0.3) (layers "F.Cu" "B.Cu") (free yes) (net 1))
 (via (at 110.014916 156.209) (size 0.6) (drill 0.3) (layers "F.Cu" "B.Cu") (free yes) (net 1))
 (segment (start 102.739916 156.839999) (end 102.739916 155.334001) (width 0.2) (layer "F.Cu") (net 6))
 (segment (start 102.739916 155.334001) (end 102.864916 155.209001) (width 0.2) (layer "F.Cu") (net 6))
 (segment (start 102.764916 158.14) (end 102.764916 156.864999) (width 0.2) (layer "F.Cu") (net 6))
 (segment (start 102.764916 156.864999) (end 102.739916 156.839999) (width 0.2) (layer "F.Cu") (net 6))
 (segment (start 102.864916 155.209001) (end 102.864916 154.864) (width 0.2) (layer "F.Cu") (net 6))
 (segment (start 102.289916 155.334001) (end 102.164916 155.209001) (width 0.2) (layer "F.Cu") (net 2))
 (segment (start 102.164916 155.209001) (end 102.164916 154.864) (width 0.2) (layer "F.Cu") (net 2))
 (segment (start 102.289916 156.839999) (end 102.289916 155.334001) (width 0.2) (layer "F.Cu") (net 2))
 (segment (start 102.264916 156.864999) (end 102.289916 156.839999) (width 0.2) (layer "F.Cu") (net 2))
 (segment (start 102.264916 158.14) (end 102.264916 156.864999) (width 0.2) (layer "F.Cu") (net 2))
 (segment (start 108.764916 156.864999) (end 108.739916 156.839999) (width 0.2) (layer "F.Cu") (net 8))
 (segment (start 108.764916 158.14) (end 108.764916 156.864999) (width 0.2) (layer "F.Cu") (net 8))
 (segment (start 108.864916 155.209001) (end 108.864916 154.864) (width 0.2) (layer "F.Cu") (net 8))
 (segment (start 108.739916 155.334001) (end 108.864916 155.209001) (width 0.2) (layer "F.Cu") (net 8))
 (segment (start 108.739916 156.839999) (end 108.739916 155.334001) (width 0.2) (layer "F.Cu") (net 8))
 (segment (start 108.164916 155.209001) (end 108.164916 154.864) (width 0.2) (layer "F.Cu") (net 4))
 (segment (start 108.264916 158.14) (end 108.264916 156.864999) (width 0.2) (layer "F.Cu") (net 4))
 (segment (start 108.264916 156.864999) (end 108.289916 156.839999) (width 0.2) (layer "F.Cu") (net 4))
 (segment (start 108.289916 156.839999) (end 108.289916 155.334001) (width 0.2) (layer "F.Cu") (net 4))
 (segment (start 108.289916 155.334001) (end 108.164916 155.209001) (width 0.2) (layer "F.Cu") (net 4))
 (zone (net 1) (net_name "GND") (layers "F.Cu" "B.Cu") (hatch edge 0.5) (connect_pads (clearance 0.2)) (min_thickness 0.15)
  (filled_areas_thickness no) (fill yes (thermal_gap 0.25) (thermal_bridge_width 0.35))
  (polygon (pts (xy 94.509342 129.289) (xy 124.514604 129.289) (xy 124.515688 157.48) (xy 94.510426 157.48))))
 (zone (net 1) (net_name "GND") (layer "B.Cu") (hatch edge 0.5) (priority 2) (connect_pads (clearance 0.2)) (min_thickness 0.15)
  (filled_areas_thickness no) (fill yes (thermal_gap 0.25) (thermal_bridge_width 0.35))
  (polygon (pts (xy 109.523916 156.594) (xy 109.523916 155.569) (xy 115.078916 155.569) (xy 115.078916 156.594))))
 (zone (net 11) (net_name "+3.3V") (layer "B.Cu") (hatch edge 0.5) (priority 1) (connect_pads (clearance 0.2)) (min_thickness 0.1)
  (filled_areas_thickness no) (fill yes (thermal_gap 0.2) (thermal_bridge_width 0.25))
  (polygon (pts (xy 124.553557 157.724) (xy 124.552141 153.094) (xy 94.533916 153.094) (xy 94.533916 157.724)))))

